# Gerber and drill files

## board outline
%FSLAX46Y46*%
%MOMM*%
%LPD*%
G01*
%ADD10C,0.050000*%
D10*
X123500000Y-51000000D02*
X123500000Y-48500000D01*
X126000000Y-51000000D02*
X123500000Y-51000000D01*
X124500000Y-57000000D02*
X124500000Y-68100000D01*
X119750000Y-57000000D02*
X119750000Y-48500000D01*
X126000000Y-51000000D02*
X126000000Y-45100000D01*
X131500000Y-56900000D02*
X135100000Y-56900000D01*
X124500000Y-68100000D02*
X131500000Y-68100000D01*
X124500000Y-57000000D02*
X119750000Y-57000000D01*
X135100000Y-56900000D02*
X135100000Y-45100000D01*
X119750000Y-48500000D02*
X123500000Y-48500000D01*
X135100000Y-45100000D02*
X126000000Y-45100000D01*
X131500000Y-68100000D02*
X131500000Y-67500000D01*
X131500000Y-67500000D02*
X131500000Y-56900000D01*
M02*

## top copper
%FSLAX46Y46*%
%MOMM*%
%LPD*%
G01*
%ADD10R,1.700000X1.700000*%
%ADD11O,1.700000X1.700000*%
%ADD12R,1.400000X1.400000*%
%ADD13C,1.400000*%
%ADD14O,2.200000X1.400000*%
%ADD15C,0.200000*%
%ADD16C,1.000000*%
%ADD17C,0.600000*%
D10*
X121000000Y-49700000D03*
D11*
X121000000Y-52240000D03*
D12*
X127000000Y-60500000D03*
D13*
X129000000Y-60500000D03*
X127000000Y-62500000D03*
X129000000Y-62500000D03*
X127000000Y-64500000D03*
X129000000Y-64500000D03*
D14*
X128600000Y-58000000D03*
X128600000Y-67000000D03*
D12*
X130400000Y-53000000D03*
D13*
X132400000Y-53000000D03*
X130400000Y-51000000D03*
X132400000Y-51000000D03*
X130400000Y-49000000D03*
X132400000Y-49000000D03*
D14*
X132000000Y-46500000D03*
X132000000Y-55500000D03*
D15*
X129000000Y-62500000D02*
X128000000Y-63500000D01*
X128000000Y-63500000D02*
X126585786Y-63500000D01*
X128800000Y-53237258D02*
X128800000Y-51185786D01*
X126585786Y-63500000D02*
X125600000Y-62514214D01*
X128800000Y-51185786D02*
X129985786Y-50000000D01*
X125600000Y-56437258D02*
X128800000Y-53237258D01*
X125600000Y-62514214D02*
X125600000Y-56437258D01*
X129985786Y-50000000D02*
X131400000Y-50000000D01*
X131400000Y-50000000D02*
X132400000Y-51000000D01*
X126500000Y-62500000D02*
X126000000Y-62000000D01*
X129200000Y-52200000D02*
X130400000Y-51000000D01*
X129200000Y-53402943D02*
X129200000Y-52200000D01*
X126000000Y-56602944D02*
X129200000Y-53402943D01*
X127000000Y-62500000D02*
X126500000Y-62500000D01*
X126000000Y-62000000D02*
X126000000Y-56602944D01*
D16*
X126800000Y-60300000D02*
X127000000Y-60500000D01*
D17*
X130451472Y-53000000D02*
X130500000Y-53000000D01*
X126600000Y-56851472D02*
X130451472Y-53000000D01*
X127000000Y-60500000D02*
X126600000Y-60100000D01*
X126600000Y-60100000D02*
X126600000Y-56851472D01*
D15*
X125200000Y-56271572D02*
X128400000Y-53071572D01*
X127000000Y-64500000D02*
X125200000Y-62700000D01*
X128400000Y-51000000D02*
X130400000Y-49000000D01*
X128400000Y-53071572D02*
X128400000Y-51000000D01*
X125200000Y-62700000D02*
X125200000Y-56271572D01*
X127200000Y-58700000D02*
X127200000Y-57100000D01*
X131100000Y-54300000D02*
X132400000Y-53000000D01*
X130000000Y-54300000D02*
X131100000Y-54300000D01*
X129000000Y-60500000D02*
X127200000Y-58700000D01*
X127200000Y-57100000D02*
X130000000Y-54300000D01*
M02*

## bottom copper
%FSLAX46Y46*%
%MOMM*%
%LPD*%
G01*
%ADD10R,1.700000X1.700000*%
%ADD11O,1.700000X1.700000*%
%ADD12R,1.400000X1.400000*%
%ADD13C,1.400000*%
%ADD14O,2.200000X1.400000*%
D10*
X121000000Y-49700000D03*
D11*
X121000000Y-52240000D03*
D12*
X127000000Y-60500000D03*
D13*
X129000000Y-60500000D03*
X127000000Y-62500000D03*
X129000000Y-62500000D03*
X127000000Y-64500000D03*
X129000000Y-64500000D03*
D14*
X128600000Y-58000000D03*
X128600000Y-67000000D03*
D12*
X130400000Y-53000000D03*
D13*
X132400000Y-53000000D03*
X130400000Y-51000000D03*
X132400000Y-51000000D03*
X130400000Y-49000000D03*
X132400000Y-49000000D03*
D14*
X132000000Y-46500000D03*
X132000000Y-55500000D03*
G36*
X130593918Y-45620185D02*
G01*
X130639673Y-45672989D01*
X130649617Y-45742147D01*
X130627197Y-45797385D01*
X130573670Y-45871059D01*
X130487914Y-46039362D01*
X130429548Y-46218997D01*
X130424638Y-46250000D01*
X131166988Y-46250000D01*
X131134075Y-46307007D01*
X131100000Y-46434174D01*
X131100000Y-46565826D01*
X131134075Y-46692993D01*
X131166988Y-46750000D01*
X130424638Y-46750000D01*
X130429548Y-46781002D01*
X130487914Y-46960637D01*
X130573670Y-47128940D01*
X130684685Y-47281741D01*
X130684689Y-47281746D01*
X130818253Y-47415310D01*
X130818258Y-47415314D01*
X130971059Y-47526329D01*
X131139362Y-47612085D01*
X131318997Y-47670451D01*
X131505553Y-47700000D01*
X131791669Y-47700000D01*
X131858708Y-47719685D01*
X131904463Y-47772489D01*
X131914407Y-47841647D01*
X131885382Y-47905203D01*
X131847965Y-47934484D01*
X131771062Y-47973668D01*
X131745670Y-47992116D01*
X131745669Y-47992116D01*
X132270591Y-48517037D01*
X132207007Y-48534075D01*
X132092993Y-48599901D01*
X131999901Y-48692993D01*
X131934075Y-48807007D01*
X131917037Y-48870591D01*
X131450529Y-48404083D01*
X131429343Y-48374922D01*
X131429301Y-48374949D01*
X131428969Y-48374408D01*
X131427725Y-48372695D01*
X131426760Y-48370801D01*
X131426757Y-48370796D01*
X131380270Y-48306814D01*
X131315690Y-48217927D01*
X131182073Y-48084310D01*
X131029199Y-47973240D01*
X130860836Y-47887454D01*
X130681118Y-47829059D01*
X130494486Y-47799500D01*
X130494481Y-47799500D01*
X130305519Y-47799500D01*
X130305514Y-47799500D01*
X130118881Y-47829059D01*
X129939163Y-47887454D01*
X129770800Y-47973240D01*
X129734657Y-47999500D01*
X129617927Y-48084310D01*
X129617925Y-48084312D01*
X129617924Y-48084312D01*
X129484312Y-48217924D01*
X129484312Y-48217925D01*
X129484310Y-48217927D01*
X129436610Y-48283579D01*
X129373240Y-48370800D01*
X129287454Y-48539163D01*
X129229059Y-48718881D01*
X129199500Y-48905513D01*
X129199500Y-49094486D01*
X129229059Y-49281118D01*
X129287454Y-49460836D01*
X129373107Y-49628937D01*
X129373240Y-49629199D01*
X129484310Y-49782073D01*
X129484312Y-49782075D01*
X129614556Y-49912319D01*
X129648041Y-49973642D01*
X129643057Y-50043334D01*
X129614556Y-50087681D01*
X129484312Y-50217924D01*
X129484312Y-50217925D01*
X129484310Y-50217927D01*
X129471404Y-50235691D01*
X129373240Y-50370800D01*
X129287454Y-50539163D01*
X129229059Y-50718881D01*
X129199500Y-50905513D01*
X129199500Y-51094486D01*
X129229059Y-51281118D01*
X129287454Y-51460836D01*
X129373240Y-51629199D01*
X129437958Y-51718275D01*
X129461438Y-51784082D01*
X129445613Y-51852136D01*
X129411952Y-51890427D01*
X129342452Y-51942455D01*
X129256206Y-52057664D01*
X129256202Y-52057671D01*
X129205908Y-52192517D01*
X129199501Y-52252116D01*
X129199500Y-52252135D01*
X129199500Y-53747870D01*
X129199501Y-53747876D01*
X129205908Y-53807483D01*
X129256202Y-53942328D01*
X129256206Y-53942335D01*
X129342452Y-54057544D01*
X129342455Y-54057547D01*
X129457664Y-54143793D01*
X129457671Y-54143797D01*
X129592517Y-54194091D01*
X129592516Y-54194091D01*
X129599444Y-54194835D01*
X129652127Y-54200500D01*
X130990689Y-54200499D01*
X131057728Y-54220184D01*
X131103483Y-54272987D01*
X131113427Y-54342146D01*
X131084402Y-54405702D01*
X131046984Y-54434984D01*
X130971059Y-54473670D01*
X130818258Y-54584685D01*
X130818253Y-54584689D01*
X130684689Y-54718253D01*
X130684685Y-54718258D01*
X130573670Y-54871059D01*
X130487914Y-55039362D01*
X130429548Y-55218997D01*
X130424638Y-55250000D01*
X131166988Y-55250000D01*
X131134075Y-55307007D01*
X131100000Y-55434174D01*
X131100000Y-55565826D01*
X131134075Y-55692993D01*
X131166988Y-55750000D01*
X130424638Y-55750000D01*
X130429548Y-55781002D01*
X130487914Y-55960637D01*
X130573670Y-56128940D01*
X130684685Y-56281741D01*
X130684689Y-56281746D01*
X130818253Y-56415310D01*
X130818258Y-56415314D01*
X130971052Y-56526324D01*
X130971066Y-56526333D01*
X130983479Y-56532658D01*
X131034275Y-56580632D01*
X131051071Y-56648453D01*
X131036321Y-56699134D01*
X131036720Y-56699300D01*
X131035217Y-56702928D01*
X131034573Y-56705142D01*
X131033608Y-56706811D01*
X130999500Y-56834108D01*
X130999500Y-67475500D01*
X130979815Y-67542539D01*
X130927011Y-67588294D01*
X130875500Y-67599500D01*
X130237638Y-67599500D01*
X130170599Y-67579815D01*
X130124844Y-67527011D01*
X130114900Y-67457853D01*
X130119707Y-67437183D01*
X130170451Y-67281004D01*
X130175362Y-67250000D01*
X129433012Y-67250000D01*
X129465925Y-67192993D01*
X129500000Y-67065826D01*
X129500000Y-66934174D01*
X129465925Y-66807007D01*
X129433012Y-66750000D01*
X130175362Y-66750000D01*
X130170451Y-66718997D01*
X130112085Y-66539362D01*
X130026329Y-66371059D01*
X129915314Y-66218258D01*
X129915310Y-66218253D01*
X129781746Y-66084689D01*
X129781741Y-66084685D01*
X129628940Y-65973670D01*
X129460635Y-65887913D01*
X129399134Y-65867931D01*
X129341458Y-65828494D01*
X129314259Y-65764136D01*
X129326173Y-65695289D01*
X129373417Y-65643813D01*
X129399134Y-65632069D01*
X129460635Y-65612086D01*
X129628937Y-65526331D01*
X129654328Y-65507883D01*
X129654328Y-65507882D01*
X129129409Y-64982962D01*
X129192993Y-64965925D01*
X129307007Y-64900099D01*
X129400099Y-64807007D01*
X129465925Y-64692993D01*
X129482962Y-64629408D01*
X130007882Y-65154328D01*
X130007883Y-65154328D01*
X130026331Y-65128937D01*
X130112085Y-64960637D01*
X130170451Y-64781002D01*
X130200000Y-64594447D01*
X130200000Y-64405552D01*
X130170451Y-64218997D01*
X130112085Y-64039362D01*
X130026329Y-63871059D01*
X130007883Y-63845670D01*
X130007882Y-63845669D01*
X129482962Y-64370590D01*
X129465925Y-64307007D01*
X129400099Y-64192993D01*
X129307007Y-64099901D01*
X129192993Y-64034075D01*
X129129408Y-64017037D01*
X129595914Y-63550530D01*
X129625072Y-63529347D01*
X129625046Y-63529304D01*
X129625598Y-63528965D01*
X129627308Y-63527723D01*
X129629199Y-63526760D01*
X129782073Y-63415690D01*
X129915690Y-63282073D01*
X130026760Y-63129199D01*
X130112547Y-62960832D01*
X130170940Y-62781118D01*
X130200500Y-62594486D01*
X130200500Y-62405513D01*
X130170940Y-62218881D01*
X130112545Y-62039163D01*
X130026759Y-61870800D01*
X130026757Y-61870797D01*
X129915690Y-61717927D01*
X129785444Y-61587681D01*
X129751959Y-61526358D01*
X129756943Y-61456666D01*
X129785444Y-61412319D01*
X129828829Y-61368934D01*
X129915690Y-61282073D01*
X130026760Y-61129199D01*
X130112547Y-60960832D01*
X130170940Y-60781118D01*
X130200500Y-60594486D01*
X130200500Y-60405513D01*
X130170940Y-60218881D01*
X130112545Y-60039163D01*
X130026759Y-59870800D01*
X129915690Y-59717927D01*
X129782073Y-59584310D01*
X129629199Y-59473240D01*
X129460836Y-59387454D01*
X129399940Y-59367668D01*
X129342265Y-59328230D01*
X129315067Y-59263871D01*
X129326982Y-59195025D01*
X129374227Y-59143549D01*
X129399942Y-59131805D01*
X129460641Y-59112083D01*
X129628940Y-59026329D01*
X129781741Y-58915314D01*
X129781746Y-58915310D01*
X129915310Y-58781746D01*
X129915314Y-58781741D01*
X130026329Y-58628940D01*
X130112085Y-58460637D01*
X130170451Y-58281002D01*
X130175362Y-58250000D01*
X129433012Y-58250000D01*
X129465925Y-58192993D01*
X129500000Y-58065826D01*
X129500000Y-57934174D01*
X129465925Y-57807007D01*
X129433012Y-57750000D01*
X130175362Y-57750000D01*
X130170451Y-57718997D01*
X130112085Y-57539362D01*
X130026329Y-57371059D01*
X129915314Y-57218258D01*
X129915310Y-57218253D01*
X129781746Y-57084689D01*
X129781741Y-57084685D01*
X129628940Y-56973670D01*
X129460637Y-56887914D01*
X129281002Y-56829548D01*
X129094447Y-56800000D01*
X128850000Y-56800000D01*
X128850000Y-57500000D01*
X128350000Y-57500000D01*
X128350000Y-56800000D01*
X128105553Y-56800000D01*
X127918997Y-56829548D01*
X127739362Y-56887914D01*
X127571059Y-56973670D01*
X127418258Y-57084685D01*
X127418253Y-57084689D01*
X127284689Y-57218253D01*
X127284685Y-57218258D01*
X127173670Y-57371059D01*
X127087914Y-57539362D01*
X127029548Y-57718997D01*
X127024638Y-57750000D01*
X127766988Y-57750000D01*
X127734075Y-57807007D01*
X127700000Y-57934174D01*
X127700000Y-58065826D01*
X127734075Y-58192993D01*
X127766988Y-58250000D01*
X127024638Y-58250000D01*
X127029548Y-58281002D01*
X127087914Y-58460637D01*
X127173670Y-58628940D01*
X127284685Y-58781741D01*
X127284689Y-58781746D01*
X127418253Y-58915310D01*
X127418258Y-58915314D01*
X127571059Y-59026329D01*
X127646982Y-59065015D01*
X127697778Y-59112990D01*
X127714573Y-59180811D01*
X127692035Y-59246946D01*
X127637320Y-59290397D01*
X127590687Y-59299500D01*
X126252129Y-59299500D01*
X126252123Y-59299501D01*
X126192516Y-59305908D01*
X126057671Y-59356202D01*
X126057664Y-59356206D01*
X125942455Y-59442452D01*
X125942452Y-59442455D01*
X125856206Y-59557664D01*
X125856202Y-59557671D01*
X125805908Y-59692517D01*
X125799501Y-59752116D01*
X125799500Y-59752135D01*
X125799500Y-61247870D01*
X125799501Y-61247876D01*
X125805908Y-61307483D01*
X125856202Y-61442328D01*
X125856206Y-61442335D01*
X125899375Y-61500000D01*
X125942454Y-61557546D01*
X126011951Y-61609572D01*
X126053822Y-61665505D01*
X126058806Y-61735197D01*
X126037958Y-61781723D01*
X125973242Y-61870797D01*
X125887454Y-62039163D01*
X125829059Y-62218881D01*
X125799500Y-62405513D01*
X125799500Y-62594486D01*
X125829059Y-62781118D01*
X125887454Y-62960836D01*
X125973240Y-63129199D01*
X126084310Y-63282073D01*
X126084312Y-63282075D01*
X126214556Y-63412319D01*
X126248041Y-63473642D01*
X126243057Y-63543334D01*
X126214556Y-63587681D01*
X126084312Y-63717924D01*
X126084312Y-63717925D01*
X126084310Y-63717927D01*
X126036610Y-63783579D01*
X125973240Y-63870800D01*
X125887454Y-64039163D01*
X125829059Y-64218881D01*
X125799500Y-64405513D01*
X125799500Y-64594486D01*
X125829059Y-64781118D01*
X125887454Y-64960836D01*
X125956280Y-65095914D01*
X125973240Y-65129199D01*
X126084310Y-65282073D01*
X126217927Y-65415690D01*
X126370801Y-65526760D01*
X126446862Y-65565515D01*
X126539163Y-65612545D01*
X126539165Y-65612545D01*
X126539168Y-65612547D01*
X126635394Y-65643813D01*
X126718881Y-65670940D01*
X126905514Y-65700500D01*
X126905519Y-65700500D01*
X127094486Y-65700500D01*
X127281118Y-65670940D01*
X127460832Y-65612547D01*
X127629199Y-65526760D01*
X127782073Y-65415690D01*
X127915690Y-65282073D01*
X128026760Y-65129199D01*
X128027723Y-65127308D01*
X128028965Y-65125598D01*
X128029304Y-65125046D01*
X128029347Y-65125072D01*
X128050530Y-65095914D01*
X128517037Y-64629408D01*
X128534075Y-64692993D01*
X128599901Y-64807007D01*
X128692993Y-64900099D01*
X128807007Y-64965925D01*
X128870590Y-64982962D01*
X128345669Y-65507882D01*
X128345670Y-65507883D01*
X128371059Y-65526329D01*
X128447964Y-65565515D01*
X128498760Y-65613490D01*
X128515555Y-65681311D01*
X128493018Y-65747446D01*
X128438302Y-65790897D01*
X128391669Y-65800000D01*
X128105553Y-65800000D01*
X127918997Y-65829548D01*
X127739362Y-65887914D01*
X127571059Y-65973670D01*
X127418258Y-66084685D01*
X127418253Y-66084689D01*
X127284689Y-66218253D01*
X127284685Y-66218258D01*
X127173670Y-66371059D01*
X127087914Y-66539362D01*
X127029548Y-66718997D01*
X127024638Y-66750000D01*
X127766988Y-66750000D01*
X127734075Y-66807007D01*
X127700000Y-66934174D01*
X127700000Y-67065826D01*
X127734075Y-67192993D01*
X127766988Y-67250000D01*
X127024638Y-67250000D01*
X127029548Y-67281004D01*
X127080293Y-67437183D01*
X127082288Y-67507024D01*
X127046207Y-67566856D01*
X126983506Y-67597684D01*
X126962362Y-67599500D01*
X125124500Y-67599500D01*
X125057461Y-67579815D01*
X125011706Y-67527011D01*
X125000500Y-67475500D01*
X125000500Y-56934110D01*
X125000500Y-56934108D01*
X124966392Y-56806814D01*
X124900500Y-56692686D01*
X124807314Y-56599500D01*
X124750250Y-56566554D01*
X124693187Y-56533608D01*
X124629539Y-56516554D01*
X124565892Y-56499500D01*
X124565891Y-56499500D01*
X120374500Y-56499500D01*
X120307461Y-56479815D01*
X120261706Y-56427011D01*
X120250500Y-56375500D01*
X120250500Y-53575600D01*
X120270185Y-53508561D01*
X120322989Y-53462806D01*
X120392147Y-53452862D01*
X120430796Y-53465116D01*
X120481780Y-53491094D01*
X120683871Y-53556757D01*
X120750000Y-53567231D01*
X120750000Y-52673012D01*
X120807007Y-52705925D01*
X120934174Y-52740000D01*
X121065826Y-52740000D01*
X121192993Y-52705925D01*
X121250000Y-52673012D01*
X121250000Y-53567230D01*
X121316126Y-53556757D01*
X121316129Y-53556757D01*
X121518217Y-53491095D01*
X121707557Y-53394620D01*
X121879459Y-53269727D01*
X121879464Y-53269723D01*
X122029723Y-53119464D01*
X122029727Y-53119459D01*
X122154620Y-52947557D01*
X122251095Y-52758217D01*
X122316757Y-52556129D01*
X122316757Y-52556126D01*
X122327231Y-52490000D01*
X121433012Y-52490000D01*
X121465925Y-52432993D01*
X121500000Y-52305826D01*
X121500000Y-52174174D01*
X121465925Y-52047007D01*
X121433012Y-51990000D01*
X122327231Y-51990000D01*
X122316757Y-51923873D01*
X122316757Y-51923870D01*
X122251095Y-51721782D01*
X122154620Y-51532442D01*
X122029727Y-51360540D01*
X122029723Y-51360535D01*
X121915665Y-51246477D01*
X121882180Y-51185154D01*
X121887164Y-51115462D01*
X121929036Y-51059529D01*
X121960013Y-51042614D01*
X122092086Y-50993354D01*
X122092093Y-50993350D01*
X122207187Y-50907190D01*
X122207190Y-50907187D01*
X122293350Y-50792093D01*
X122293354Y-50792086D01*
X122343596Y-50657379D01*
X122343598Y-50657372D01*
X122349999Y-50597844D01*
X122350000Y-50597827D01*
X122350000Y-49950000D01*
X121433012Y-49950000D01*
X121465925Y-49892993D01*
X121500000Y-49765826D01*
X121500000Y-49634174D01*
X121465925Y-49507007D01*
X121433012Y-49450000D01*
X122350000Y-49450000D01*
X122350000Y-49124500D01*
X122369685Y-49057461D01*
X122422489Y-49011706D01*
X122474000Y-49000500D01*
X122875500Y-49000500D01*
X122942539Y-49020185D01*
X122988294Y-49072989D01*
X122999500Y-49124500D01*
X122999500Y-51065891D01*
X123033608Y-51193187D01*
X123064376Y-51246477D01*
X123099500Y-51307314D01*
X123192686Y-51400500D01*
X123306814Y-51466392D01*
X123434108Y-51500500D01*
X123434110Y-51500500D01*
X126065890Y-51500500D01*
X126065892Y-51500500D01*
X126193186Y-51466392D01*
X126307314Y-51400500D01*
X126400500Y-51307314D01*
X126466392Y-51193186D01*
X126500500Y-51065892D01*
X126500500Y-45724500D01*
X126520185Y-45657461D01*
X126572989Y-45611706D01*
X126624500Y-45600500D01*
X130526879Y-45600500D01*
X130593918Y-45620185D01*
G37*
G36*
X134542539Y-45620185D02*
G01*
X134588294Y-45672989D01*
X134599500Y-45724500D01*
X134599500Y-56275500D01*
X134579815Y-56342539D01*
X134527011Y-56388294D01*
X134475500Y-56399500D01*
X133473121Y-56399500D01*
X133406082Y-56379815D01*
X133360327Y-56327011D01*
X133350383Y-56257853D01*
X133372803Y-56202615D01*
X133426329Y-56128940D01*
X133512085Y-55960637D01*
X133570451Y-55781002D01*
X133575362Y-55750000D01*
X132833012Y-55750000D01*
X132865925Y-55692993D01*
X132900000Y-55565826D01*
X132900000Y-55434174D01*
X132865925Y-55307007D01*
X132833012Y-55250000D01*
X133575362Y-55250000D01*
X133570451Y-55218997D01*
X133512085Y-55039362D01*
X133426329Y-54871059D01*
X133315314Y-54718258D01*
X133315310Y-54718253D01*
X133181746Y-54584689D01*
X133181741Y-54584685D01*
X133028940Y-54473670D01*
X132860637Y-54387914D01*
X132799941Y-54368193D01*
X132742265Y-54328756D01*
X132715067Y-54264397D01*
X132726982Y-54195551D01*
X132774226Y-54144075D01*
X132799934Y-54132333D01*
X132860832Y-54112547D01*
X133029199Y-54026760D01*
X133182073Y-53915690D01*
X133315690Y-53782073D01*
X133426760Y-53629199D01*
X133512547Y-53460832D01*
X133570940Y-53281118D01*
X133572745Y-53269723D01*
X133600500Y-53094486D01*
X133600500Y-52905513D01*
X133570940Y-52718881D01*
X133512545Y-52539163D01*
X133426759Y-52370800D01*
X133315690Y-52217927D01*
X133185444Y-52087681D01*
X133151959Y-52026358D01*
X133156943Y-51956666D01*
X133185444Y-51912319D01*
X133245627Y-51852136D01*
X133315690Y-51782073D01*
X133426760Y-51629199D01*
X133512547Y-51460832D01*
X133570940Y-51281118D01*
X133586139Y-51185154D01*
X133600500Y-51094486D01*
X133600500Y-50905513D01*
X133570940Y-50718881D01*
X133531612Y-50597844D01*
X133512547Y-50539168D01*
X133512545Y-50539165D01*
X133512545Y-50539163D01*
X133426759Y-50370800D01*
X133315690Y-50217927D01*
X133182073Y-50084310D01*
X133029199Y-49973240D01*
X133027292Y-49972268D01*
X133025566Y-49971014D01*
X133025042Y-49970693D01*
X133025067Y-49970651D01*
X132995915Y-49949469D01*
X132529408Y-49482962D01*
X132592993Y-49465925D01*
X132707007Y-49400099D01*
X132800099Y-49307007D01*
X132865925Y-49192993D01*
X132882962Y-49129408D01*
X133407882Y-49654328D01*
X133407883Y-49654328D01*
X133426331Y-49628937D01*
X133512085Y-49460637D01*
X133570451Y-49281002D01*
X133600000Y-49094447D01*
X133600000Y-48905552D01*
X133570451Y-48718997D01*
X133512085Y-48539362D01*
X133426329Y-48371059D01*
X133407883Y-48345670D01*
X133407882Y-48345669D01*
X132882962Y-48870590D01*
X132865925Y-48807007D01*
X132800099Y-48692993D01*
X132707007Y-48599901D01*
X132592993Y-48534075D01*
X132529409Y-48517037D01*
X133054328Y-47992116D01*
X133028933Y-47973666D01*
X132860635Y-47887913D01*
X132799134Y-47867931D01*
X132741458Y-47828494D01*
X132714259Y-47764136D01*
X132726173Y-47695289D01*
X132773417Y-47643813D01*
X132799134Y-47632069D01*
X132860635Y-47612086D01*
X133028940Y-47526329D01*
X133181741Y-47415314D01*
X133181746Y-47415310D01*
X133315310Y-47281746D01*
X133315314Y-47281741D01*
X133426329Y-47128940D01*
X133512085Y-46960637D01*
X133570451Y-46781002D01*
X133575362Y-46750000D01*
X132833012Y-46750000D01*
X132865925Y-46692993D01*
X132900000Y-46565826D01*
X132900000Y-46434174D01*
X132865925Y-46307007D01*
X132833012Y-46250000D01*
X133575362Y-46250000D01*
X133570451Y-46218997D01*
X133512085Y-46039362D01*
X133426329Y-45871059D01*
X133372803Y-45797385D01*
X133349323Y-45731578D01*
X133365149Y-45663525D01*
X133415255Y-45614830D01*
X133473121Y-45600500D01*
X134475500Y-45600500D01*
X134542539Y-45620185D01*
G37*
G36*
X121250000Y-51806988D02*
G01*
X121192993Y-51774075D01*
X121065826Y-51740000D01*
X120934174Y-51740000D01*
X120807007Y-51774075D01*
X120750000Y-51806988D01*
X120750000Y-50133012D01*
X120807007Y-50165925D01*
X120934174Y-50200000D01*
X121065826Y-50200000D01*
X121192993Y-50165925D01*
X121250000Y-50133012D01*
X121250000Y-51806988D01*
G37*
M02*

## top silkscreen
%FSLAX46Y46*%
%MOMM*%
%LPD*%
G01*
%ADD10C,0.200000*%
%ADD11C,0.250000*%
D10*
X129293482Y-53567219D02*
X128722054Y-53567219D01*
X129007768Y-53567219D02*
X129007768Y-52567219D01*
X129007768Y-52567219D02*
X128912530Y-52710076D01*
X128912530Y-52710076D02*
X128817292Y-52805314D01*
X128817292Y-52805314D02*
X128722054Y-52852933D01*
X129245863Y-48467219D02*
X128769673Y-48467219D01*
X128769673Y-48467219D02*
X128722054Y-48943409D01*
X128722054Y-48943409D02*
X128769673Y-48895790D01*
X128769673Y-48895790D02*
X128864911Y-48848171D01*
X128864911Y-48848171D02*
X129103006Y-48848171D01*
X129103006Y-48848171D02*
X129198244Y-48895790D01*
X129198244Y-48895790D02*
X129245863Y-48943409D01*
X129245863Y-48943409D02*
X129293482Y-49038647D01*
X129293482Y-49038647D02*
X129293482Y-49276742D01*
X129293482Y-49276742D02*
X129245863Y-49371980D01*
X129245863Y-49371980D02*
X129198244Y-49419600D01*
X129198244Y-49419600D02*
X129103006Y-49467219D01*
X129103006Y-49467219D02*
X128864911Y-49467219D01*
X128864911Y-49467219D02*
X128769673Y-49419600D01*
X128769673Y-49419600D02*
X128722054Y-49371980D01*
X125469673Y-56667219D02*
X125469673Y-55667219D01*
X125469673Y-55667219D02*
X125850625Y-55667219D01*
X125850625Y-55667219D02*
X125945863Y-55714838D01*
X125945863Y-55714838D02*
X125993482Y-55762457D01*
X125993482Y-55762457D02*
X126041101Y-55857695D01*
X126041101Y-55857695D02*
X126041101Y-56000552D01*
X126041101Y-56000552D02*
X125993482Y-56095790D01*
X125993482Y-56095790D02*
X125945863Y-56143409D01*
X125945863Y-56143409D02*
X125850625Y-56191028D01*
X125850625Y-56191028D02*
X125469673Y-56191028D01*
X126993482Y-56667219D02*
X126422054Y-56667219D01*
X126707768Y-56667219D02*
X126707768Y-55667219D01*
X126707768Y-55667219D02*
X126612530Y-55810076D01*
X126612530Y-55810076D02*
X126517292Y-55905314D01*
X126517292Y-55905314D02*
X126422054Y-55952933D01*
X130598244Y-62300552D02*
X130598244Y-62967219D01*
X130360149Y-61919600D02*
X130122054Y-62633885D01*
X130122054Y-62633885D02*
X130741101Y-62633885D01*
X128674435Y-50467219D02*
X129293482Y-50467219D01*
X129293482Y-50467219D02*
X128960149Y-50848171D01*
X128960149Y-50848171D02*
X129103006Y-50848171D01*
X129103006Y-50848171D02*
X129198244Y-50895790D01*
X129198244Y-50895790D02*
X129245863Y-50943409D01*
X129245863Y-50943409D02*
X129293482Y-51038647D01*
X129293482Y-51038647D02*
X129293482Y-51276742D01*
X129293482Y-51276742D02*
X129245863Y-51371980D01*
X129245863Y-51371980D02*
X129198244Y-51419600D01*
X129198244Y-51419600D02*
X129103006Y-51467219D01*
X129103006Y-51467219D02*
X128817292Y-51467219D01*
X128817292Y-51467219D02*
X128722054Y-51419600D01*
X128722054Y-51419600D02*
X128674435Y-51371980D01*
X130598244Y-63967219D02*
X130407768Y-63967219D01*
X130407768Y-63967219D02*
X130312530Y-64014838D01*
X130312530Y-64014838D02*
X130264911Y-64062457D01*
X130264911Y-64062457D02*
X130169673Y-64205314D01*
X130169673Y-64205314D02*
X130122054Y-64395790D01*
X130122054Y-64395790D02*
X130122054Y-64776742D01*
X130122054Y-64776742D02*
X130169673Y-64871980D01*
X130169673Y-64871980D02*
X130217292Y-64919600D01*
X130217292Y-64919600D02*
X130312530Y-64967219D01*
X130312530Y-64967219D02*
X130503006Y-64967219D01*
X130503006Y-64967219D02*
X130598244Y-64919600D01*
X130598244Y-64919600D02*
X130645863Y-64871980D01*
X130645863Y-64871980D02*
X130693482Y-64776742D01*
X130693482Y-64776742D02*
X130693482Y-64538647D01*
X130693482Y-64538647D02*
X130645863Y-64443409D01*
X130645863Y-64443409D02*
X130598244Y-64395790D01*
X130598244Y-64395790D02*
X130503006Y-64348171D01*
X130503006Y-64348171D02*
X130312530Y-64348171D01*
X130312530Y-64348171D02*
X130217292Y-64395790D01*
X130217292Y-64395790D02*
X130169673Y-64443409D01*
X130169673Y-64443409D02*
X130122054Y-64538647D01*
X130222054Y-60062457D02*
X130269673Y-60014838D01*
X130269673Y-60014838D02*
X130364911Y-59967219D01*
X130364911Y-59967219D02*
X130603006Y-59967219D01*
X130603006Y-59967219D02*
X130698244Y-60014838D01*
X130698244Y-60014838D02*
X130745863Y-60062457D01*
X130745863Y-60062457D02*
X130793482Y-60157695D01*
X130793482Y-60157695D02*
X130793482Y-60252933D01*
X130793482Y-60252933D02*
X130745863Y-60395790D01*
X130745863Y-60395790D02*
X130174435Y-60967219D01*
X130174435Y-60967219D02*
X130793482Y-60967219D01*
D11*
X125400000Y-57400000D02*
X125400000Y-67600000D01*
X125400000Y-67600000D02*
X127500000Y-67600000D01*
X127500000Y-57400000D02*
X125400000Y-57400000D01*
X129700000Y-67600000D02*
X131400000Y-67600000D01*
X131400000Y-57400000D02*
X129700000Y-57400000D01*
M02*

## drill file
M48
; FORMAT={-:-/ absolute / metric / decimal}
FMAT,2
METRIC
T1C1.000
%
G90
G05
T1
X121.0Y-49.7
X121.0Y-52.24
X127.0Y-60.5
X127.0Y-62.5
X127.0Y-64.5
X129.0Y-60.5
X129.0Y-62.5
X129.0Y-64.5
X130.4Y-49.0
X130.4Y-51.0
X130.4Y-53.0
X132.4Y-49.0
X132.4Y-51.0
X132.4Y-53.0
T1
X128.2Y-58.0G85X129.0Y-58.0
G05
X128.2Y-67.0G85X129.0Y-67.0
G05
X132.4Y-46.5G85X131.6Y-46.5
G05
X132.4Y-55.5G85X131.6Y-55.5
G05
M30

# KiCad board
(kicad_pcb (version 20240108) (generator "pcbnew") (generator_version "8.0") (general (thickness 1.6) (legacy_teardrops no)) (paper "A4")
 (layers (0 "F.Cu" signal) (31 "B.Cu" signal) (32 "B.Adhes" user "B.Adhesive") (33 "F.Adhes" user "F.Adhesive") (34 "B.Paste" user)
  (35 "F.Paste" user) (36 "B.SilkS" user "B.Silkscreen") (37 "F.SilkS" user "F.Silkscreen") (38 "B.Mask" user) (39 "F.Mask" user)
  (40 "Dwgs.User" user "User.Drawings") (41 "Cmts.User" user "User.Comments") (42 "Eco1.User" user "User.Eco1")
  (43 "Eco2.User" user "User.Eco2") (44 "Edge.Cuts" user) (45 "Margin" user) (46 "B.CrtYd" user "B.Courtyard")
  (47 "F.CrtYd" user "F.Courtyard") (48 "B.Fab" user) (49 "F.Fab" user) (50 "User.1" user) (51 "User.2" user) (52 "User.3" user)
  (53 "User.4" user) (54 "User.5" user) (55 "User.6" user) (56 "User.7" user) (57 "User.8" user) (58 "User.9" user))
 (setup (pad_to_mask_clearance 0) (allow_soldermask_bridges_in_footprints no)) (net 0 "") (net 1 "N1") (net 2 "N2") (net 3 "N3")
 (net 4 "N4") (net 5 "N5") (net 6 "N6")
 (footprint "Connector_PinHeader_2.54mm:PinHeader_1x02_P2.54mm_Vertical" (layer "F.Cu") (at 121 49.7)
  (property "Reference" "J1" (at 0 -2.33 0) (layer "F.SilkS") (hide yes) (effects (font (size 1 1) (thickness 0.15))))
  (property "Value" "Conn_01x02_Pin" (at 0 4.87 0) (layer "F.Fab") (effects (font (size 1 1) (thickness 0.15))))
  (pad "1" thru_hole rect (at 0 0) (size 1.7 1.7) (drill 1) (layers "*.Cu" "*.Mask") (remove_unused_layers no) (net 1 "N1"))
  (pad "2" thru_hole oval (at 0 2.54) (size 1.7 1.7) (drill 1) (layers "*.Cu" "*.Mask") (remove_unused_layers no) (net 1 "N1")))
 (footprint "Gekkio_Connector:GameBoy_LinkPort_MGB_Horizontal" (layer "F.Cu") (at 127 60.5)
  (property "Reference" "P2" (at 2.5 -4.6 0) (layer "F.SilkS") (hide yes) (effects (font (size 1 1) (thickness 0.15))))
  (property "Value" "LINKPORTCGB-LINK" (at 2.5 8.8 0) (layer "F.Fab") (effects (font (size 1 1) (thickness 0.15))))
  (fp_line (start -1.6 -3.1) (end -1.6 7.1) (stroke (width 0.25) (type solid)) (layer "F.SilkS"))
  (fp_line (start -1.6 7.1) (end 0.5 7.1) (stroke (width 0.25) (type solid)) (layer "F.SilkS"))
  (fp_line (start 0.5 -3.1) (end -1.6 -3.1) (stroke (width 0.25) (type solid)) (layer "F.SilkS"))
  (fp_line (start 2.7 7.1) (end 4.4 7.1) (stroke (width 0.25) (type solid)) (layer "F.SilkS"))
  (fp_line (start 4.4 -3.1) (end 2.7 -3.1) (stroke (width 0.25) (type solid)) (layer "F.SilkS"))
  (pad "1" thru_hole rect (at 0 0) (size 1.4 1.4) (drill 1) (layers "*.Cu" "*.Mask") (remove_unused_layers no) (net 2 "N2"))
  (pad "2" thru_hole circle (at 2 0) (size 1.4 1.4) (drill 1) (layers "*.Cu" "*.Mask") (remove_unused_layers no) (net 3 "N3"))
  (pad "3" thru_hole circle (at 0 2) (size 1.4 1.4) (drill 1) (layers "*.Cu" "*.Mask") (remove_unused_layers no) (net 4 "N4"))
  (pad "4" thru_hole circle (at 2 2) (size 1.4 1.4) (drill 1) (layers "*.Cu" "*.Mask") (remove_unused_layers no) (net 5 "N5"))
  (pad "5" thru_hole circle (at 0 4) (size 1.4 1.4) (drill 1) (layers "*.Cu" "*.Mask") (remove_unused_layers no) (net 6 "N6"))
  (pad "6" thru_hole circle (at 2 4) (size 1.4 1.4) (drill 1) (layers "*.Cu" "*.Mask") (remove_unused_layers no) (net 1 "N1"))
  (pad "SH" thru_hole oval (at 1.6 -2.5 90) (size 1.4 2.2) (drill oval 1 1.8) (layers "*.Cu" "*.Mask") (remove_unused_layers no)
   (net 1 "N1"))
  (pad "SH" thru_hole oval (at 1.6 6.5 90) (size 1.4 2.2) (drill oval 1 1.8) (layers "*.Cu" "*.Mask") (remove_unused_layers no) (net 1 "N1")))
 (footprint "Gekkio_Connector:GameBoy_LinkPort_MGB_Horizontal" (layer "B.Cu") (at 130.4 53)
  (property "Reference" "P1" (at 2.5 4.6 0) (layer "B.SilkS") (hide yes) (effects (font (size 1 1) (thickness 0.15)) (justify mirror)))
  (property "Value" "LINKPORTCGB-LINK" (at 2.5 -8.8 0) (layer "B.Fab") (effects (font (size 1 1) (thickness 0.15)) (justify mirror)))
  (pad "1" thru_hole rect (at 0 0) (size 1.4 1.4) (drill 1) (layers "*.Cu" "*.Mask") (remove_unused_layers no) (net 2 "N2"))
  (pad "2" thru_hole circle (at 2 0) (size 1.4 1.4) (drill 1) (layers "*.Cu" "*.Mask") (remove_unused_layers no) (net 3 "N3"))
  (pad "3" thru_hole circle (at 0 -2) (size 1.4 1.4) (drill 1) (layers "*.Cu" "*.Mask") (remove_unused_layers no) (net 4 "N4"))
  (pad "4" thru_hole circle (at 2 -2) (size 1.4 1.4) (drill 1) (layers "*.Cu" "*.Mask") (remove_unused_layers no) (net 5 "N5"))
  (pad "5" thru_hole circle (at 0 -4) (size 1.4 1.4) (drill 1) (layers "*.Cu" "*.Mask") (remove_unused_layers no) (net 6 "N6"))
  (pad "6" thru_hole circle (at 2 -4) (size 1.4 1.4) (drill 1) (layers "*.Cu" "*.Mask") (remove_unused_layers no) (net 1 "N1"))
  (pad "SH" thru_hole oval (at 1.6 -6.5 270) (size 1.4 2.2) (drill oval 1 1.8) (layers "*.Cu" "*.Mask") (remove_unused_layers no)
   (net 1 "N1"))
  (pad "SH" thru_hole oval (at 1.6 2.5 270) (size 1.4 2.2) (drill oval 1 1.8) (layers "*.Cu" "*.Mask") (remove_unused_layers no)
   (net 1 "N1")))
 (gr_line (start 123.5 51) (end 123.5 48.5) (stroke (width 0.05) (type default)) (layer "Edge.Cuts"))
 (gr_line (start 126 51) (end 123.5 51) (stroke (width 0.05) (type default)) (layer "Edge.Cuts"))
 (gr_line (start 124.5 57) (end 124.5 68.1) (stroke (width 0.05) (type default)) (layer "Edge.Cuts"))
 (gr_line (start 119.75 57) (end 119.75 48.5) (stroke (width 0.05) (type default)) (layer "Edge.Cuts"))
 (gr_line (start 126 51) (end 126 45.1) (stroke (width 0.05) (type default)) (layer "Edge.Cuts"))
 (gr_line (start 131.5 56.9) (end 135.1 56.9) (stroke (width 0.05) (type default)) (layer "Edge.Cuts"))
 (gr_line (start 124.5 68.1) (end 131.5 68.1) (stroke (width 0.05) (type default)) (layer "Edge.Cuts"))
 (gr_line (start 124.5 57) (end 119.75 57) (stroke (width 0.05) (type default)) (layer "Edge.Cuts"))
 (gr_line (start 135.1 56.9) (end 135.1 45.1) (stroke (width 0.05) (type default)) (layer "Edge.Cuts"))
 (gr_line (start 119.75 48.5) (end 123.5 48.5) (stroke (width 0.05) (type default)) (layer "Edge.Cuts"))
 (gr_line (start 135.1 45.1) (end 126 45.1) (stroke (width 0.05) (type default)) (layer "Edge.Cuts"))
 (gr_line (start 131.5 68.1) (end 131.5 67.5) (stroke (width 0.05) (type default)) (layer "Edge.Cuts"))
 (gr_line (start 131.5 67.5) (end 131.5 56.9) (stroke (width 0.05) (type default)) (layer "Edge.Cuts"))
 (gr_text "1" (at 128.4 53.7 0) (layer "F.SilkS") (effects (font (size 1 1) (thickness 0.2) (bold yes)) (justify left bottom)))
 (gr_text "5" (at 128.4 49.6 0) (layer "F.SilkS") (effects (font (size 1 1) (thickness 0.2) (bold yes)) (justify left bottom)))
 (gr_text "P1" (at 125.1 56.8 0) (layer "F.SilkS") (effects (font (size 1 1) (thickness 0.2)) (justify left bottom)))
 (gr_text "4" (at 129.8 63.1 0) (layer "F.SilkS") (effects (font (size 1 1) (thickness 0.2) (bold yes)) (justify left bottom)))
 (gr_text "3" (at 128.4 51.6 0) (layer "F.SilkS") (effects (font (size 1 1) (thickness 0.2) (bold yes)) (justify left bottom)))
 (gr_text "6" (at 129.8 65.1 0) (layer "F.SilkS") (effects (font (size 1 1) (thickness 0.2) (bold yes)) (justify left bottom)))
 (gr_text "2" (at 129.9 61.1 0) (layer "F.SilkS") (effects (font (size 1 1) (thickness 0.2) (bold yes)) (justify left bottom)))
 (segment (start 129 62.5) (end 128 63.5) (width 0.2) (layer "F.Cu") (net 5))
 (segment (start 128 63.5) (end 126.585786 63.5) (width 0.2) (layer "F.Cu") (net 5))
 (segment (start 128.8 53.237258) (end 128.8 51.185786) (width 0.2) (layer "F.Cu") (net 5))
 (segment (start 126.585786 63.5) (end 125.6 62.514214) (width 0.2) (layer "F.Cu") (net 5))
 (segment (start 128.8 51.185786) (end 129.985786 50) (width 0.2) (layer "F.Cu") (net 5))
 (segment (start 125.6 56.437258) (end 128.8 53.237258) (width 0.2) (layer "F.Cu") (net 5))
 (segment (start 125.6 62.514214) (end 125.6 56.437258) (width 0.2) (layer "F.Cu") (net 5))
 (segment (start 129.985786 50) (end 131.4 50) (width 0.2) (layer "F.Cu") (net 5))
 (segment (start 131.4 50) (end 132.4 51) (width 0.2) (layer "F.Cu") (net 5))
 (segment (start 126.5 62.5) (end 126 62) (width 0.2) (layer "F.Cu") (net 4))
 (segment (start 129.2 52.2) (end 130.4 51) (width 0.2) (layer "F.Cu") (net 4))
 (segment (start 129.2 53.402943) (end 129.2 52.2) (width 0.2) (layer "F.Cu") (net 4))
 (segment (start 126 56.602944) (end 129.2 53.402943) (width 0.2) (layer "F.Cu") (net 4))
 (segment (start 127 62.5) (end 126.5 62.5) (width 0.2) (layer "F.Cu") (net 4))
 (segment (start 126 62) (end 126 56.602944) (width 0.2) (layer "F.Cu") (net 4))
 (segment (start 126.8 60.3) (end 127 60.5) (width 1) (layer "F.Cu") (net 2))
 (segment (start 130.451472 53) (end 130.5 53) (width 0.6) (layer "F.Cu") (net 2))
 (segment (start 126.6 56.851472) (end 130.451472 53) (width 0.6) (layer "F.Cu") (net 2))
 (segment (start 127 60.5) (end 126.6 60.1) (width 0.6) (layer "F.Cu") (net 2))
 (segment (start 126.6 60.1) (end 126.6 56.851472) (width 0.6) (layer "F.Cu") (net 2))
 (segment (start 125.2 56.271572) (end 128.4 53.071572) (width 0.2) (layer "F.Cu") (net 6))
 (segment (start 127 64.5) (end 125.2 62.7) (width 0.2) (layer "F.Cu") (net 6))
 (segment (start 128.4 51) (end 130.4 49) (width 0.2) (layer "F.Cu") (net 6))
 (segment (start 128.4 53.071572) (end 128.4 51) (width 0.2) (layer "F.Cu") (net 6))
 (segment (start 125.2 62.7) (end 125.2 56.271572) (width 0.2) (layer "F.Cu") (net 6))
 (segment (start 127.2 58.7) (end 127.2 57.1) (width 0.2) (layer "F.Cu") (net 3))
 (segment (start 131.1 54.3) (end 132.4 53) (width 0.2) (layer "F.Cu") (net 3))
 (segment (start 130 54.3) (end 131.1 54.3) (width 0.2) (layer "F.Cu") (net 3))
 (segment (start 129 60.5) (end 127.2 58.7) (width 0.2) (layer "F.Cu") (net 3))
 (segment (start 127.2 57.1) (end 130 54.3) (width 0.2) (layer "F.Cu") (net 3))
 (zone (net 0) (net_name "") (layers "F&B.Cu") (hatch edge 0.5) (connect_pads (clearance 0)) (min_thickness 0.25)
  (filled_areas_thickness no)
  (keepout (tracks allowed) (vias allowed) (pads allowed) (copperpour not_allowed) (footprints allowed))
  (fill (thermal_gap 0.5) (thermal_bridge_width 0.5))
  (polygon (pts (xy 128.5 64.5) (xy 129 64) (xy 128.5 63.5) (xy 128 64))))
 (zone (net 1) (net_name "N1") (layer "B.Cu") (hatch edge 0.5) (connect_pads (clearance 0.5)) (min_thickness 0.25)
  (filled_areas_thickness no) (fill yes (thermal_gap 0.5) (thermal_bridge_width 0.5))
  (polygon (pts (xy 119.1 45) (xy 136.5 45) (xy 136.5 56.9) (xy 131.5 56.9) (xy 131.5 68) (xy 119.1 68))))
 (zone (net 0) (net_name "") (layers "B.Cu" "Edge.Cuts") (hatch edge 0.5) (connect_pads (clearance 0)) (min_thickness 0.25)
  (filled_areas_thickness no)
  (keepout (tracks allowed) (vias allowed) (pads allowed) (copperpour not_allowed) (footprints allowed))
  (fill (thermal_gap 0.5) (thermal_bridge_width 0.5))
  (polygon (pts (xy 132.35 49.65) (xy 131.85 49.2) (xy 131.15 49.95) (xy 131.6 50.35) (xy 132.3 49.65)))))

